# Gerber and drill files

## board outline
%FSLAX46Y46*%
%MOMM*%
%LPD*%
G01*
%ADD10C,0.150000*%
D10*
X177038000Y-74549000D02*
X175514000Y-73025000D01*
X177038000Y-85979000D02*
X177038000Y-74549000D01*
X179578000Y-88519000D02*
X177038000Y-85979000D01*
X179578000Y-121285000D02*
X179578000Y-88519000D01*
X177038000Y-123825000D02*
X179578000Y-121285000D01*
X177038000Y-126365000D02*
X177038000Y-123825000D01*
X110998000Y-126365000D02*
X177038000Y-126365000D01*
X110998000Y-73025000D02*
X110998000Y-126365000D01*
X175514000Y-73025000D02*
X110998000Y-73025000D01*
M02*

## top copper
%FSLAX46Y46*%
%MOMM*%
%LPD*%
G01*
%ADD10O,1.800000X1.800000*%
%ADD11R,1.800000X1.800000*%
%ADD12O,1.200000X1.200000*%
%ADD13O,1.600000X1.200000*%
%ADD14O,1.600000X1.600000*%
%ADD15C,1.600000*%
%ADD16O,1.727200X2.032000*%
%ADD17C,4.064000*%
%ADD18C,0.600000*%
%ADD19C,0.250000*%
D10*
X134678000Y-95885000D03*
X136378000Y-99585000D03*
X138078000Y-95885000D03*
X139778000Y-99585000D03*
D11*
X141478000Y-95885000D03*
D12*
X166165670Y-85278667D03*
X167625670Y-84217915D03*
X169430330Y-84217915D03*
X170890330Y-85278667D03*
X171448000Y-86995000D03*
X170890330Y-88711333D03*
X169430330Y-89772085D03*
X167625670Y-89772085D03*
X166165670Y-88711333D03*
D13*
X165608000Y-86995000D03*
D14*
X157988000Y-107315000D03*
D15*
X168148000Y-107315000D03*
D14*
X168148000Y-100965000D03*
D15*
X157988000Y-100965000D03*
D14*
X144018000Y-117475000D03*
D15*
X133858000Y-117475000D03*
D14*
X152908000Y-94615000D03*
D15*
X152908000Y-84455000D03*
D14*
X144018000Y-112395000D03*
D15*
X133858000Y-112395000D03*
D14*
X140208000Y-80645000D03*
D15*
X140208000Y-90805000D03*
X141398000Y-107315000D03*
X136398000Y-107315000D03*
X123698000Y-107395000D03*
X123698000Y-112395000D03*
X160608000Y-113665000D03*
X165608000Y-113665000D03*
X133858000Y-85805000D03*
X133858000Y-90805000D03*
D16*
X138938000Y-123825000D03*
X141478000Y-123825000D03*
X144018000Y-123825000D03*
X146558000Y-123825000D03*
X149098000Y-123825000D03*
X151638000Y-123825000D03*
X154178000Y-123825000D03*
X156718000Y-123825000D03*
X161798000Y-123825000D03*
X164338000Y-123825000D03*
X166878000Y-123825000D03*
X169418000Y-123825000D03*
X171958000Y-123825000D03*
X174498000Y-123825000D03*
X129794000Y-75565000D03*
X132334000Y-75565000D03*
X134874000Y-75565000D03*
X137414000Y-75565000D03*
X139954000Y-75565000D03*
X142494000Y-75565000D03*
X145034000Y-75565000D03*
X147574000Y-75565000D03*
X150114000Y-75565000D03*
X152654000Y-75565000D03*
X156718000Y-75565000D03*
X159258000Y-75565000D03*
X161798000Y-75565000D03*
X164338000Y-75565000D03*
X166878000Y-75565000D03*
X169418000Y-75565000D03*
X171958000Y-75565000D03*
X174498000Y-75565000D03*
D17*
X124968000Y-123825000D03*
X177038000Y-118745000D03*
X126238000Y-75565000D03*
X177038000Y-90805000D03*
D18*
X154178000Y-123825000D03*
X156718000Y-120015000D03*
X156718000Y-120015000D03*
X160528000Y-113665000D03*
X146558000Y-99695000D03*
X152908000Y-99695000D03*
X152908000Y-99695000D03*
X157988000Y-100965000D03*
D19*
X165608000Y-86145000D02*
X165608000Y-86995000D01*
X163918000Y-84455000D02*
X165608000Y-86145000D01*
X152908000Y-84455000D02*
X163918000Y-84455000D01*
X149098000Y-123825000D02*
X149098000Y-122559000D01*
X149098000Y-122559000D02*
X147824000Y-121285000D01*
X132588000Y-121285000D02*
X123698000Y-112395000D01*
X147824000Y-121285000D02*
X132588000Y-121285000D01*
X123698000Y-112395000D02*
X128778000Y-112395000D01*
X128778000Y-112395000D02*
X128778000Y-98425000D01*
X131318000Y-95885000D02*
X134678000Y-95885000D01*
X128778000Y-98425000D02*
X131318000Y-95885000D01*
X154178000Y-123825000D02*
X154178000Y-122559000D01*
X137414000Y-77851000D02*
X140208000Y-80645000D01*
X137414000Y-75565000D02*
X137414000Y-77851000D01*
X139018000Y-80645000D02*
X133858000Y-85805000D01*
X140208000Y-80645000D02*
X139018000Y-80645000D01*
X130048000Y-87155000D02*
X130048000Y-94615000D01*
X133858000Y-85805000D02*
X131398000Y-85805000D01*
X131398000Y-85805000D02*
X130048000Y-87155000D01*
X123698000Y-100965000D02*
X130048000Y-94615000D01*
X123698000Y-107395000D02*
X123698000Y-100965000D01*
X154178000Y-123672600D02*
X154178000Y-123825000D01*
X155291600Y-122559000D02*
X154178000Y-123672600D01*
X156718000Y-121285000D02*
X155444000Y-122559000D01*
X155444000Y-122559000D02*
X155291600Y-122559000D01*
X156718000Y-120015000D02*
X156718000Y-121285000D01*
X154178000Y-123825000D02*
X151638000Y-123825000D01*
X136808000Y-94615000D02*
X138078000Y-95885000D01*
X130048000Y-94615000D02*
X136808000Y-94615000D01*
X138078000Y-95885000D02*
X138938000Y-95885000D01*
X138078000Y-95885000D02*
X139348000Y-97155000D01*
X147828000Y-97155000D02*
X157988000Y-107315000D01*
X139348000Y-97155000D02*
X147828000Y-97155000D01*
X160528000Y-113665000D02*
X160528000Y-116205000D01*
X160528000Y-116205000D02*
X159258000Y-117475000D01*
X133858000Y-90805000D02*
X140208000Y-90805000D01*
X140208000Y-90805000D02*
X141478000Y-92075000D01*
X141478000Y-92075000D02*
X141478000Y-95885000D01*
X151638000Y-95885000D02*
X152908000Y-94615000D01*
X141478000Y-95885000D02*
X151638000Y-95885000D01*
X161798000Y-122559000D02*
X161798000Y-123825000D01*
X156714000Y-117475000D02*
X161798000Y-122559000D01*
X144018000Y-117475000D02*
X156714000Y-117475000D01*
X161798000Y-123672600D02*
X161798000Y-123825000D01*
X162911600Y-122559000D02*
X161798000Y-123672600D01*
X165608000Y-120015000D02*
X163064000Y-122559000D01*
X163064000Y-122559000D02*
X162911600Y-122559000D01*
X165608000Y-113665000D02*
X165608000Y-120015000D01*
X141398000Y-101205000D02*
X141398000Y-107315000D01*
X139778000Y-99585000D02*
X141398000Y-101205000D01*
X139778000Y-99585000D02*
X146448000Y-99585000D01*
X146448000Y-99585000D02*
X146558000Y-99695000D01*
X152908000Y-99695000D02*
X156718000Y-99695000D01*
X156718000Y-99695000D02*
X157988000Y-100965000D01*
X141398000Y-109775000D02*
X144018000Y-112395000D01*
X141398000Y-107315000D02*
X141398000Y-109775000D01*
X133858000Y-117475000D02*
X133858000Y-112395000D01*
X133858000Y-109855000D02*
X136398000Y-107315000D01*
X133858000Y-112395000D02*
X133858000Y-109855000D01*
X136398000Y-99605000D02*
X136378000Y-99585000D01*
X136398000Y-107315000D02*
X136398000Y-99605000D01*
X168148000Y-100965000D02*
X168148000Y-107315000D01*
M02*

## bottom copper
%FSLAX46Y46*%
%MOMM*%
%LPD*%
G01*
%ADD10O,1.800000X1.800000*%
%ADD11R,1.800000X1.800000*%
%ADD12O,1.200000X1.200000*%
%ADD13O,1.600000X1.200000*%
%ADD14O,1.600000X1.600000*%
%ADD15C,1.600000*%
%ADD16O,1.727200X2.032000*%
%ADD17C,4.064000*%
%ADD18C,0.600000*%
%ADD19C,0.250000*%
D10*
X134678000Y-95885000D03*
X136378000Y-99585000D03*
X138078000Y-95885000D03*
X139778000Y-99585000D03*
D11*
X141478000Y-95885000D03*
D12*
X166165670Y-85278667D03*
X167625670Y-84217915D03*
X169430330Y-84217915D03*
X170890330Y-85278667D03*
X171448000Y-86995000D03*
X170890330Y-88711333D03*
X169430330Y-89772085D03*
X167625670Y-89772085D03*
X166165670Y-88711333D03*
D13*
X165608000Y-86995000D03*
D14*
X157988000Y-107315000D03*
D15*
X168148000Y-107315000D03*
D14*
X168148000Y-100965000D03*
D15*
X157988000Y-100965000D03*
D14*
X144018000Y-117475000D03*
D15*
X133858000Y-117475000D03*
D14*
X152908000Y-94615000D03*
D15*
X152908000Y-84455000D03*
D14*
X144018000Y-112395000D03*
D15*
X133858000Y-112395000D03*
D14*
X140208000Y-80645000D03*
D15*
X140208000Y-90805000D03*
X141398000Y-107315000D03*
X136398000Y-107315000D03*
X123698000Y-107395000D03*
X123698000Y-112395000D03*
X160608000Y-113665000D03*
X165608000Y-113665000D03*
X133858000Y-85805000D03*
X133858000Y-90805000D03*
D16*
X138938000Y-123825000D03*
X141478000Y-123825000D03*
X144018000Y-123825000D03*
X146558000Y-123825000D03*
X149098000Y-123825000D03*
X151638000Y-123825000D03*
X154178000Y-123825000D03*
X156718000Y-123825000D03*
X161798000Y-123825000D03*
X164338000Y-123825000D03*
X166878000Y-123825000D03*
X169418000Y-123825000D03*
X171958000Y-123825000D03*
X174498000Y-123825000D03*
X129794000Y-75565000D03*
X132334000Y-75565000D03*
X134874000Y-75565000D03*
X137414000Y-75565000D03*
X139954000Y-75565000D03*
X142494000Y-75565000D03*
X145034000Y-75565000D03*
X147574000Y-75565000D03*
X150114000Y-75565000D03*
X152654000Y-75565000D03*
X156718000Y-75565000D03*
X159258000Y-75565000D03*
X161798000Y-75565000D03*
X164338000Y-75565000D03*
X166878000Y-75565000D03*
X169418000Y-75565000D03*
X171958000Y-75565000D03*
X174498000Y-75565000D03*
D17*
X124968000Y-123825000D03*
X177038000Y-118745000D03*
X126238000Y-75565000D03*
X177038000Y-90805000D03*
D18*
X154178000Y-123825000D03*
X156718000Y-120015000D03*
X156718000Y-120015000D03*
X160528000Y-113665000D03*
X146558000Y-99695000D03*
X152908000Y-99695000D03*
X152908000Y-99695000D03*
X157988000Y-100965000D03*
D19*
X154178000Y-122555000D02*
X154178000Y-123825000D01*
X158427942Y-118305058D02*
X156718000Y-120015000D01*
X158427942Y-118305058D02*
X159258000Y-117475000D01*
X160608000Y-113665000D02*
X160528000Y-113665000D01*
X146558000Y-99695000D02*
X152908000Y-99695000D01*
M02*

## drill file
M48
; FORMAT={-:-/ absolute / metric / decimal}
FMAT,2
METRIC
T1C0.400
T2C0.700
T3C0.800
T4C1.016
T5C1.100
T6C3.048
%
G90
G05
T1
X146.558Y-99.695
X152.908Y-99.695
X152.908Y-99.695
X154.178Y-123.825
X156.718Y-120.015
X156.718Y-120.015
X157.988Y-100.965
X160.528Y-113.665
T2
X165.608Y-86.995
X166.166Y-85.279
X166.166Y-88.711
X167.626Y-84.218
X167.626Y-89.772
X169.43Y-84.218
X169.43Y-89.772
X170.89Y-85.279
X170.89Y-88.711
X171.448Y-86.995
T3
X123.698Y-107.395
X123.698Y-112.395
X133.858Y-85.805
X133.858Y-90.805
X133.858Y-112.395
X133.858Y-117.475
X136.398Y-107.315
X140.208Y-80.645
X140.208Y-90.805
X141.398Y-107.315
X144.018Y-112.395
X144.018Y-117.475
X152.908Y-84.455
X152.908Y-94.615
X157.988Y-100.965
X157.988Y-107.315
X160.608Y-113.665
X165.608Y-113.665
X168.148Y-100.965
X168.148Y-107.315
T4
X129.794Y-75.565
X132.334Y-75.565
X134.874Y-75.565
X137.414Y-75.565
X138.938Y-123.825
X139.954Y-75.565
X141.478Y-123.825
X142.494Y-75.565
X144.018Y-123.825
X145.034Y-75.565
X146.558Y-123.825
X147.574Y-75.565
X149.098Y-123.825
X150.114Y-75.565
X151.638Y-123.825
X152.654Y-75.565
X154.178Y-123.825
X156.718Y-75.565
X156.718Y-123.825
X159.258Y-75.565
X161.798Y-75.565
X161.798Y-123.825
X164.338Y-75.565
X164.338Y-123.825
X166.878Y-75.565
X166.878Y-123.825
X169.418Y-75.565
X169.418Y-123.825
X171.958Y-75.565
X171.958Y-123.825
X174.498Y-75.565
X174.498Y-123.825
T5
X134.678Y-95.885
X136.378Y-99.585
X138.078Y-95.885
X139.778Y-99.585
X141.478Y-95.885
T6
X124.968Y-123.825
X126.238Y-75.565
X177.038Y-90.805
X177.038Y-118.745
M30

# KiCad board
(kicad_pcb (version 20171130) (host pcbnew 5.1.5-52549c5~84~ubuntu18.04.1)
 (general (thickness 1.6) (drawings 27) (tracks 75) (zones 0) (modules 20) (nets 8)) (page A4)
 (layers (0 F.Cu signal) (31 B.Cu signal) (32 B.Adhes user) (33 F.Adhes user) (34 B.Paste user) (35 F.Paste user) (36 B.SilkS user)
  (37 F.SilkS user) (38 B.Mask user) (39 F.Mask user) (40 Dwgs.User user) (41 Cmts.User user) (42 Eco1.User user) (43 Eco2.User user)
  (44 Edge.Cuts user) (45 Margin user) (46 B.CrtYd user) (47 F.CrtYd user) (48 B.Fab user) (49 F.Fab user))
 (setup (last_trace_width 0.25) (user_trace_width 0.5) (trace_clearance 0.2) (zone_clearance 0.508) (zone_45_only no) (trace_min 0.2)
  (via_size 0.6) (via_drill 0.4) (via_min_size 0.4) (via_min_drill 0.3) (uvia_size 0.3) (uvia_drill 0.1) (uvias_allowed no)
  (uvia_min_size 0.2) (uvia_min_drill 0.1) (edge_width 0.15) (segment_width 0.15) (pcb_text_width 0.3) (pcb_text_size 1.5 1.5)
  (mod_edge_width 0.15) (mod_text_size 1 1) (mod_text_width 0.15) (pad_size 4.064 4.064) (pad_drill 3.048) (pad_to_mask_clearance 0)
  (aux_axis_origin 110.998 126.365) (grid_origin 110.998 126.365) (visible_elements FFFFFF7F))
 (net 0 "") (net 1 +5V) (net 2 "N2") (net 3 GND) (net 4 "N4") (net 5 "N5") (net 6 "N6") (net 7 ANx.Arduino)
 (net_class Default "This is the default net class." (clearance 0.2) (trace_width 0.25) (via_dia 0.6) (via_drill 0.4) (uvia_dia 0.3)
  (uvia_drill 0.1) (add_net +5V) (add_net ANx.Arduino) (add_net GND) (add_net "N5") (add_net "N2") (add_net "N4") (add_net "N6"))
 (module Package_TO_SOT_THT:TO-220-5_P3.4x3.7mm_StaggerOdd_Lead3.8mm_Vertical (layer F.Cu) (at 141.478 95.885 180)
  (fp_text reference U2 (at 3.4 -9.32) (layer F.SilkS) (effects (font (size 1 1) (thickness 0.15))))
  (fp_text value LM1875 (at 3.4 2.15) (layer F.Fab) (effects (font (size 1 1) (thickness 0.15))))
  (pad 5 thru_hole oval (at 6.8 0 180) (size 1.8 1.8) (drill 1.1) (layers *.Cu *.Mask) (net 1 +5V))
  (pad 4 thru_hole oval (at 5.1 -3.7 180) (size 1.8 1.8) (drill 1.1) (layers *.Cu *.Mask) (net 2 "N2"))
  (pad 3 thru_hole oval (at 3.4 0 180) (size 1.8 1.8) (drill 1.1) (layers *.Cu *.Mask) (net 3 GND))
  (pad 2 thru_hole oval (at 1.7 -3.7 180) (size 1.8 1.8) (drill 1.1) (layers *.Cu *.Mask) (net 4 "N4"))
  (pad 1 thru_hole rect (at 0 0 180) (size 1.8 1.8) (drill 1.1) (layers *.Cu *.Mask) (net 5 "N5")))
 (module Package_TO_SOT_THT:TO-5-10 (layer F.Cu) (at 165.608 86.995)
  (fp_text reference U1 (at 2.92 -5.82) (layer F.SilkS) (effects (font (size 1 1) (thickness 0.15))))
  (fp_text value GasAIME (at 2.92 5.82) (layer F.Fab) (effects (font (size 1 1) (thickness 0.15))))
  (pad 10 thru_hole oval (at 0.55767 -1.716333) (size 1.2 1.2) (drill 0.7) (layers *.Cu *.Mask))
  (pad 9 thru_hole oval (at 2.01767 -2.777085) (size 1.2 1.2) (drill 0.7) (layers *.Cu *.Mask))
  (pad 8 thru_hole oval (at 3.82233 -2.777085) (size 1.2 1.2) (drill 0.7) (layers *.Cu *.Mask))
  (pad 7 thru_hole oval (at 5.28233 -1.716333) (size 1.2 1.2) (drill 0.7) (layers *.Cu *.Mask))
  (pad 6 thru_hole oval (at 5.84 0) (size 1.2 1.2) (drill 0.7) (layers *.Cu *.Mask))
  (pad 5 thru_hole oval (at 5.28233 1.716333) (size 1.2 1.2) (drill 0.7) (layers *.Cu *.Mask))
  (pad 4 thru_hole oval (at 3.82233 2.777085) (size 1.2 1.2) (drill 0.7) (layers *.Cu *.Mask))
  (pad 3 thru_hole oval (at 2.01767 2.777085) (size 1.2 1.2) (drill 0.7) (layers *.Cu *.Mask))
  (pad 2 thru_hole oval (at 0.55767 1.716333) (size 1.2 1.2) (drill 0.7) (layers *.Cu *.Mask))
  (pad 1 thru_hole oval (at 0 0) (size 1.6 1.2) (drill 0.7) (layers *.Cu *.Mask)))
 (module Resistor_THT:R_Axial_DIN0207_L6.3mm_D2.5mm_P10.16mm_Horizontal (layer F.Cu) (at 168.148 107.315 180)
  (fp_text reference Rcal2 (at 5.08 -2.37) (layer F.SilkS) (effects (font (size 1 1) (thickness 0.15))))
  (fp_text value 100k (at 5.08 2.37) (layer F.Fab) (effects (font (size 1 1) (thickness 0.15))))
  (pad 2 thru_hole oval (at 10.16 0 180) (size 1.6 1.6) (drill 0.8) (layers *.Cu *.Mask) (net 3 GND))
  (pad 1 thru_hole circle (at 0 0 180) (size 1.6 1.6) (drill 0.8) (layers *.Cu *.Mask) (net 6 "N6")))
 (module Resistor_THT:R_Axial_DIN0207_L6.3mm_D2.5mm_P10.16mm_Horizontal (layer F.Cu) (at 157.988 100.965)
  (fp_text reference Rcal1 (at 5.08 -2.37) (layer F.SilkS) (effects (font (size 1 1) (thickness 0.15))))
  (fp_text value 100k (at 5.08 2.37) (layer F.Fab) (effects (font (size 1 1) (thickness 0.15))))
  (pad 2 thru_hole oval (at 10.16 0) (size 1.6 1.6) (drill 0.8) (layers *.Cu *.Mask) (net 6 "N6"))
  (pad 1 thru_hole circle (at 0 0) (size 1.6 1.6) (drill 0.8) (layers *.Cu *.Mask) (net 4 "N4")))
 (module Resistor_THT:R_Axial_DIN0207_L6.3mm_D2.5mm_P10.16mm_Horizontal (layer F.Cu) (at 133.858 117.475)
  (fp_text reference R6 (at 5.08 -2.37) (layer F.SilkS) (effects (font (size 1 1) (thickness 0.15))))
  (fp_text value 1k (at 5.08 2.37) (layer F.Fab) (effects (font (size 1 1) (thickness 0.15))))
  (pad 2 thru_hole oval (at 10.16 0) (size 1.6 1.6) (drill 0.8) (layers *.Cu *.Mask) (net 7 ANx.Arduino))
  (pad 1 thru_hole circle (at 0 0) (size 1.6 1.6) (drill 0.8) (layers *.Cu *.Mask) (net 2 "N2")))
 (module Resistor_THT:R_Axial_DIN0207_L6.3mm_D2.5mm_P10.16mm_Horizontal (layer F.Cu) (at 152.908 84.455 270)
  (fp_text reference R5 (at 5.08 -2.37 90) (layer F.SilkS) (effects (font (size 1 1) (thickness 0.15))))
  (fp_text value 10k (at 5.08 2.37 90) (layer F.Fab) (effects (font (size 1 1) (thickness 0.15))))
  (pad 2 thru_hole oval (at 10.16 0 270) (size 1.6 1.6) (drill 0.8) (layers *.Cu *.Mask) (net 5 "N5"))
  (pad 1 thru_hole circle (at 0 0 270) (size 1.6 1.6) (drill 0.8) (layers *.Cu *.Mask)))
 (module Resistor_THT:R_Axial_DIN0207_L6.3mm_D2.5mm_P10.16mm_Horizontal (layer F.Cu) (at 133.858 112.395)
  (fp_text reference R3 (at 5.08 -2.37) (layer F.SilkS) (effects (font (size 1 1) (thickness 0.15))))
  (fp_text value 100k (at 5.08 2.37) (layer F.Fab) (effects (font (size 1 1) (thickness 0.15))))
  (pad 2 thru_hole oval (at 10.16 0) (size 1.6 1.6) (drill 0.8) (layers *.Cu *.Mask) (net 4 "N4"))
  (pad 1 thru_hole circle (at 0 0) (size 1.6 1.6) (drill 0.8) (layers *.Cu *.Mask) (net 2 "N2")))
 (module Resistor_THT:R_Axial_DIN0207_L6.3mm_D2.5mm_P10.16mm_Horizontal (layer F.Cu) (at 140.208 90.805 90)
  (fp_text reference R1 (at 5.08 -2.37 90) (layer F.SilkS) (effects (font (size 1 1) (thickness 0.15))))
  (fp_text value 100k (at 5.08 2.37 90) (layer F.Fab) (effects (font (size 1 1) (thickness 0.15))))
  (pad 2 thru_hole oval (at 10.16 0 90) (size 1.6 1.6) (drill 0.8) (layers *.Cu *.Mask) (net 3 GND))
  (pad 1 thru_hole circle (at 0 0 90) (size 1.6 1.6) (drill 0.8) (layers *.Cu *.Mask) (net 5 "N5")))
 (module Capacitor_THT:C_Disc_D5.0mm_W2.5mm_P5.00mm (layer F.Cu) (at 136.398 107.315)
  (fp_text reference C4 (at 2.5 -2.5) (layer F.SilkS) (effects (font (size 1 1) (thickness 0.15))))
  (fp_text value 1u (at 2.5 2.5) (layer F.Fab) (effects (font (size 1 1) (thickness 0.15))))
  (pad 2 thru_hole circle (at 5 0) (size 1.6 1.6) (drill 0.8) (layers *.Cu *.Mask) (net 4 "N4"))
  (pad 1 thru_hole circle (at 0 0) (size 1.6 1.6) (drill 0.8) (layers *.Cu *.Mask) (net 2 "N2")))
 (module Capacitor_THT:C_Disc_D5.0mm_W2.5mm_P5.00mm (layer F.Cu) (at 123.698 112.395 90)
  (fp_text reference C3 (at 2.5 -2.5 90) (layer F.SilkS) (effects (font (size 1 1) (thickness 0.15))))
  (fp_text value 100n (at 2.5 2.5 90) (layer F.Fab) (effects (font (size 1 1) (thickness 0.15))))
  (pad 2 thru_hole circle (at 5 0 90) (size 1.6 1.6) (drill 0.8) (layers *.Cu *.Mask) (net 3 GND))
  (pad 1 thru_hole circle (at 0 0 90) (size 1.6 1.6) (drill 0.8) (layers *.Cu *.Mask) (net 1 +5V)))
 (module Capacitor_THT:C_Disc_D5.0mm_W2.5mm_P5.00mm (layer F.Cu) (at 165.608 113.665 180)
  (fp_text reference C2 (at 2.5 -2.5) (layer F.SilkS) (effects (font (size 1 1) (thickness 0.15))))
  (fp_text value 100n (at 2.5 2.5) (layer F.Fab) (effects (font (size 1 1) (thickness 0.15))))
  (pad 2 thru_hole circle (at 5 0 180) (size 1.6 1.6) (drill 0.8) (layers *.Cu *.Mask) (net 3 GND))
  (pad 1 thru_hole circle (at 0 0 180) (size 1.6 1.6) (drill 0.8) (layers *.Cu *.Mask) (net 7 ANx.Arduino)))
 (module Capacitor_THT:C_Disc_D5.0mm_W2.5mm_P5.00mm (layer F.Cu) (at 133.858 90.805 90)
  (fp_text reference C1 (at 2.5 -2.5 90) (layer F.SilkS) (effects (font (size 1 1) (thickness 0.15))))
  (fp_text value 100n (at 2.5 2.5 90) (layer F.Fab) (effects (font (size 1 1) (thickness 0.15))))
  (pad 2 thru_hole circle (at 5 0 90) (size 1.6 1.6) (drill 0.8) (layers *.Cu *.Mask) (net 3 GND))
  (pad 1 thru_hole circle (at 0 0 90) (size 1.6 1.6) (drill 0.8) (layers *.Cu *.Mask) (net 5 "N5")))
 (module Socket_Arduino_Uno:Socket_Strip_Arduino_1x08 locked (layer F.Cu) (at 138.938 123.825)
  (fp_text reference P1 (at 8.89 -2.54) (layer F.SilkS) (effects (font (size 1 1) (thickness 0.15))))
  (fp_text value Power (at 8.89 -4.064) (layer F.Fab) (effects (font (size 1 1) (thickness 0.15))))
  (pad 1 thru_hole oval (at 0 0) (size 1.7272 2.032) (drill 1.016) (layers *.Cu *.Mask F.SilkS))
  (pad 2 thru_hole oval (at 2.54 0) (size 1.7272 2.032) (drill 1.016) (layers *.Cu *.Mask F.SilkS))
  (pad 3 thru_hole oval (at 5.08 0) (size 1.7272 2.032) (drill 1.016) (layers *.Cu *.Mask F.SilkS))
  (pad 4 thru_hole oval (at 7.62 0) (size 1.7272 2.032) (drill 1.016) (layers *.Cu *.Mask F.SilkS))
  (pad 5 thru_hole oval (at 10.16 0) (size 1.7272 2.032) (drill 1.016) (layers *.Cu *.Mask F.SilkS) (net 1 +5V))
  (pad 6 thru_hole oval (at 12.7 0) (size 1.7272 2.032) (drill 1.016) (layers *.Cu *.Mask F.SilkS) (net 3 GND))
  (pad 7 thru_hole oval (at 15.24 0) (size 1.7272 2.032) (drill 1.016) (layers *.Cu *.Mask F.SilkS) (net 3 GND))
  (pad 8 thru_hole oval (at 17.78 0) (size 1.7272 2.032) (drill 1.016) (layers *.Cu *.Mask F.SilkS)))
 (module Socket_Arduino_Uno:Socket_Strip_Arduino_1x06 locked (layer F.Cu) (at 161.798 123.825)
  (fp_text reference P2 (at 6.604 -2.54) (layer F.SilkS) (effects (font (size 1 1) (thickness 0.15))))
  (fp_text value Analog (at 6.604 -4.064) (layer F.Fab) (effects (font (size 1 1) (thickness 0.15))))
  (pad 1 thru_hole oval (at 0 0) (size 1.7272 2.032) (drill 1.016) (layers *.Cu *.Mask F.SilkS) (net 7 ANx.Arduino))
  (pad 2 thru_hole oval (at 2.54 0) (size 1.7272 2.032) (drill 1.016) (layers *.Cu *.Mask F.SilkS))
  (pad 3 thru_hole oval (at 5.08 0) (size 1.7272 2.032) (drill 1.016) (layers *.Cu *.Mask F.SilkS))
  (pad 4 thru_hole oval (at 7.62 0) (size 1.7272 2.032) (drill 1.016) (layers *.Cu *.Mask F.SilkS))
  (pad 5 thru_hole oval (at 10.16 0) (size 1.7272 2.032) (drill 1.016) (layers *.Cu *.Mask F.SilkS))
  (pad 6 thru_hole oval (at 12.7 0) (size 1.7272 2.032) (drill 1.016) (layers *.Cu *.Mask F.SilkS)))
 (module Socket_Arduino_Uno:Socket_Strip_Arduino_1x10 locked (layer F.Cu) (at 129.794 75.565)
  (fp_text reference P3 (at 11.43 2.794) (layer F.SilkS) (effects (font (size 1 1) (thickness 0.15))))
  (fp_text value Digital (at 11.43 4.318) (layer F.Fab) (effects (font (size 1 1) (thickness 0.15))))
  (pad 1 thru_hole oval (at 0 0) (size 1.7272 2.032) (drill 1.016) (layers *.Cu *.Mask F.SilkS))
  (pad 2 thru_hole oval (at 2.54 0) (size 1.7272 2.032) (drill 1.016) (layers *.Cu *.Mask F.SilkS))
  (pad 3 thru_hole oval (at 5.08 0) (size 1.7272 2.032) (drill 1.016) (layers *.Cu *.Mask F.SilkS))
  (pad 4 thru_hole oval (at 7.62 0) (size 1.7272 2.032) (drill 1.016) (layers *.Cu *.Mask F.SilkS) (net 3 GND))
  (pad 5 thru_hole oval (at 10.16 0) (size 1.7272 2.032) (drill 1.016) (layers *.Cu *.Mask F.SilkS))
  (pad 6 thru_hole oval (at 12.7 0) (size 1.7272 2.032) (drill 1.016) (layers *.Cu *.Mask F.SilkS))
  (pad 7 thru_hole oval (at 15.24 0) (size 1.7272 2.032) (drill 1.016) (layers *.Cu *.Mask F.SilkS))
  (pad 8 thru_hole oval (at 17.78 0) (size 1.7272 2.032) (drill 1.016) (layers *.Cu *.Mask F.SilkS))
  (pad 9 thru_hole oval (at 20.32 0) (size 1.7272 2.032) (drill 1.016) (layers *.Cu *.Mask F.SilkS))
  (pad 10 thru_hole oval (at 22.86 0) (size 1.7272 2.032) (drill 1.016) (layers *.Cu *.Mask F.SilkS)))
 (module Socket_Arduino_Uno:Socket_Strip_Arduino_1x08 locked (layer F.Cu) (at 156.718 75.565)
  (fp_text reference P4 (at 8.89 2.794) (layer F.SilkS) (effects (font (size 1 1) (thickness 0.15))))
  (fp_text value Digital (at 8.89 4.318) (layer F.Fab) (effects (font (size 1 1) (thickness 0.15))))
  (pad 1 thru_hole oval (at 0 0) (size 1.7272 2.032) (drill 1.016) (layers *.Cu *.Mask F.SilkS))
  (pad 2 thru_hole oval (at 2.54 0) (size 1.7272 2.032) (drill 1.016) (layers *.Cu *.Mask F.SilkS))
  (pad 3 thru_hole oval (at 5.08 0) (size 1.7272 2.032) (drill 1.016) (layers *.Cu *.Mask F.SilkS))
  (pad 4 thru_hole oval (at 7.62 0) (size 1.7272 2.032) (drill 1.016) (layers *.Cu *.Mask F.SilkS))
  (pad 5 thru_hole oval (at 10.16 0) (size 1.7272 2.032) (drill 1.016) (layers *.Cu *.Mask F.SilkS))
  (pad 6 thru_hole oval (at 12.7 0) (size 1.7272 2.032) (drill 1.016) (layers *.Cu *.Mask F.SilkS))
  (pad 7 thru_hole oval (at 15.24 0) (size 1.7272 2.032) (drill 1.016) (layers *.Cu *.Mask F.SilkS))
  (pad 8 thru_hole oval (at 17.78 0) (size 1.7272 2.032) (drill 1.016) (layers *.Cu *.Mask F.SilkS)))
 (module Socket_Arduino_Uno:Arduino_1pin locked (layer F.Cu) (at 124.968 123.825)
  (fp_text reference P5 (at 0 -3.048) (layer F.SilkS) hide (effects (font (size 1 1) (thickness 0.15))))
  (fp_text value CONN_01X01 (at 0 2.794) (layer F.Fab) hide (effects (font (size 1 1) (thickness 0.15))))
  (pad 1 thru_hole circle (at 0 0) (size 4.064 4.064) (drill 3.048) (layers *.Cu *.Mask F.SilkS)))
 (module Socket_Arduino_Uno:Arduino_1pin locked (layer F.Cu) (at 177.038 118.745)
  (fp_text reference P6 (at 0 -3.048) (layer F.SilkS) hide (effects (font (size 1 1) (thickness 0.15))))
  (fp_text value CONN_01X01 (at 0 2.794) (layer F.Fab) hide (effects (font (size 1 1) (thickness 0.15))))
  (pad 1 thru_hole circle (at 0 0) (size 4.064 4.064) (drill 3.048) (layers *.Cu *.Mask F.SilkS)))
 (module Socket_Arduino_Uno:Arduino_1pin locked (layer F.Cu) (at 126.238 75.565)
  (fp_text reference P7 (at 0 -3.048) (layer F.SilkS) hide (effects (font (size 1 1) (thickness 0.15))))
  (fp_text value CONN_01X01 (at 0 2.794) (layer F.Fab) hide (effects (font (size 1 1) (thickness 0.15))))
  (pad 1 thru_hole circle (at 0 0) (size 4.064 4.064) (drill 3.048) (layers *.Cu *.Mask F.SilkS)))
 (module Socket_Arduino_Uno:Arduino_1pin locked (layer F.Cu) (at 177.038 90.805)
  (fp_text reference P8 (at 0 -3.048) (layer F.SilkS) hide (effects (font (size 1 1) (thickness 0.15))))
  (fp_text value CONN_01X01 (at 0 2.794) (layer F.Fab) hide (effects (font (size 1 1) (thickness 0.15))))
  (pad 1 thru_hole circle (at 0 0) (size 4.064 4.064) (drill 3.048) (layers *.Cu *.Mask F.SilkS)))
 (gr_line (start 177.038 74.549) (end 175.514 73.025) (angle 90) (layer Edge.Cuts) (width 0.15))
 (gr_line (start 177.038 85.979) (end 177.038 74.549) (angle 90) (layer Edge.Cuts) (width 0.15))
 (gr_line (start 179.578 88.519) (end 177.038 85.979) (angle 90) (layer Edge.Cuts) (width 0.15))
 (gr_line (start 179.578 121.285) (end 179.578 88.519) (angle 90) (layer Edge.Cuts) (width 0.15))
 (gr_line (start 177.038 123.825) (end 179.578 121.285) (angle 90) (layer Edge.Cuts) (width 0.15))
 (gr_line (start 177.038 126.365) (end 177.038 123.825) (angle 90) (layer Edge.Cuts) (width 0.15))
 (gr_line (start 110.998 126.365) (end 177.038 126.365) (angle 90) (layer Edge.Cuts) (width 0.15))
 (gr_line (start 110.998 73.025) (end 110.998 126.365) (angle 90) (layer Edge.Cuts) (width 0.15))
 (gr_line (start 175.514 73.025) (end 110.998 73.025) (angle 90) (layer Edge.Cuts) (width 0.15))
 (segment (start 165.608 86.145) (end 165.608 86.995) (width 0.25) (layer F.Cu) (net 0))
 (segment (start 163.918 84.455) (end 165.608 86.145) (width 0.25) (layer F.Cu) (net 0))
 (segment (start 152.908 84.455) (end 163.918 84.455) (width 0.25) (layer F.Cu) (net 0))
 (segment (start 149.098 123.825) (end 149.098 122.559) (width 0.25) (layer F.Cu) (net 1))
 (segment (start 149.098 122.559) (end 147.824 121.285) (width 0.25) (layer F.Cu) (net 1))
 (segment (start 132.588 121.285) (end 123.698 112.395) (width 0.25) (layer F.Cu) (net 1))
 (segment (start 147.824 121.285) (end 132.588 121.285) (width 0.25) (layer F.Cu) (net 1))
 (segment (start 123.698 112.395) (end 128.778 112.395) (width 0.25) (layer F.Cu) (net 1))
 (segment (start 128.778 112.395) (end 128.778 98.425) (width 0.25) (layer F.Cu) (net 1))
 (segment (start 131.318 95.885) (end 134.678 95.885) (width 0.25) (layer F.Cu) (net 1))
 (segment (start 128.778 98.425) (end 131.318 95.885) (width 0.25) (layer F.Cu) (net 1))
 (segment (start 154.178 123.825) (end 154.178 122.559) (width 0.25) (layer F.Cu) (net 3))
 (segment (start 137.414 77.851) (end 140.208 80.645) (width 0.25) (layer F.Cu) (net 3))
 (segment (start 137.414 75.565) (end 137.414 77.851) (width 0.25) (layer F.Cu) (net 3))
 (segment (start 139.018 80.645) (end 133.858 85.805) (width 0.25) (layer F.Cu) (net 3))
 (segment (start 140.208 80.645) (end 139.018 80.645) (width 0.25) (layer F.Cu) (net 3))
 (segment (start 130.048 87.155) (end 130.048 94.615) (width 0.25) (layer F.Cu) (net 3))
 (segment (start 133.858 85.805) (end 131.398 85.805) (width 0.25) (layer F.Cu) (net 3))
 (segment (start 131.398 85.805) (end 130.048 87.155) (width 0.25) (layer F.Cu) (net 3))
 (segment (start 123.698 100.965) (end 130.048 94.615) (width 0.25) (layer F.Cu) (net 3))
 (segment (start 123.698 107.395) (end 123.698 100.965) (width 0.25) (layer F.Cu) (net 3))
 (segment (start 154.178 122.555) (end 154.178 123.825) (width 0.25) (layer B.Cu) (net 3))
 (via (at 154.178 123.825) (size 0.6) (drill 0.4) (layers F.Cu B.Cu) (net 3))
 (segment (start 158.427942 118.305058) (end 156.718 120.015) (width 0.25) (layer B.Cu) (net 3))
 (via (at 156.718 120.015) (size 0.6) (drill 0.4) (layers F.Cu B.Cu) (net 3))
 (via (at 156.718 120.015) (size 0.6) (drill 0.4) (layers F.Cu B.Cu) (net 3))
 (segment (start 154.178 123.6726) (end 154.178 123.825) (width 0.25) (layer F.Cu) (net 3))
 (segment (start 155.2916 122.559) (end 154.178 123.6726) (width 0.25) (layer F.Cu) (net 3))
 (segment (start 156.718 121.285) (end 155.444 122.559) (width 0.25) (layer F.Cu) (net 3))
 (segment (start 155.444 122.559) (end 155.2916 122.559) (width 0.25) (layer F.Cu) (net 3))
 (segment (start 156.718 120.015) (end 156.718 121.285) (width 0.25) (layer F.Cu) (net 3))
 (segment (start 154.178 123.825) (end 151.638 123.825) (width 0.25) (layer F.Cu) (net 3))
 (segment (start 136.808 94.615) (end 138.078 95.885) (width 0.25) (layer F.Cu) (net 3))
 (segment (start 130.048 94.615) (end 136.808 94.615) (width 0.25) (layer F.Cu) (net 3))
 (segment (start 138.078 95.885) (end 138.938 95.885) (width 0.25) (layer F.Cu) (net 3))
 (segment (start 138.078 95.885) (end 139.348 97.155) (width 0.25) (layer F.Cu) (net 3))
 (segment (start 147.828 97.155) (end 157.988 107.315) (width 0.25) (layer F.Cu) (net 3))
 (segment (start 139.348 97.155) (end 147.828 97.155) (width 0.25) (layer F.Cu) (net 3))
 (segment (start 158.427942 118.305058) (end 159.258 117.475) (width 0.25) (layer B.Cu) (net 3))
 (via (at 160.528 113.665) (size 0.6) (drill 0.4) (layers F.Cu B.Cu) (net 3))
 (segment (start 160.608 113.665) (end 160.528 113.665) (width 0.25) (layer B.Cu) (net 3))
 (segment (start 160.528 113.665) (end 160.528 116.205) (width 0.25) (layer F.Cu) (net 3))
 (segment (start 160.528 116.205) (end 159.258 117.475) (width 0.25) (layer F.Cu) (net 3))
 (segment (start 133.858 90.805) (end 140.208 90.805) (width 0.25) (layer F.Cu) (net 5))
 (segment (start 140.208 90.805) (end 141.478 92.075) (width 0.25) (layer F.Cu) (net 5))
 (segment (start 141.478 92.075) (end 141.478 95.885) (width 0.25) (layer F.Cu) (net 5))
 (segment (start 151.638 95.885) (end 152.908 94.615) (width 0.25) (layer F.Cu) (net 5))
 (segment (start 141.478 95.885) (end 151.638 95.885) (width 0.25) (layer F.Cu) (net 5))
 (segment (start 161.798 122.559) (end 161.798 123.825) (width 0.25) (layer F.Cu) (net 7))
 (segment (start 156.714 117.475) (end 161.798 122.559) (width 0.25) (layer F.Cu) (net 7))
 (segment (start 144.018 117.475) (end 156.714 117.475) (width 0.25) (layer F.Cu) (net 7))
 (segment (start 161.798 123.6726) (end 161.798 123.825) (width 0.25) (layer F.Cu) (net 7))
 (segment (start 162.9116 122.559) (end 161.798 123.6726) (width 0.25) (layer F.Cu) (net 7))
 (segment (start 165.608 120.015) (end 163.064 122.559) (width 0.25) (layer F.Cu) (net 7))
 (segment (start 163.064 122.559) (end 162.9116 122.559) (width 0.25) (layer F.Cu) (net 7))
 (segment (start 165.608 113.665) (end 165.608 120.015) (width 0.25) (layer F.Cu) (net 7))
 (segment (start 141.398 101.205) (end 141.398 107.315) (width 0.25) (layer F.Cu) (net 4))
 (segment (start 139.778 99.585) (end 141.398 101.205) (width 0.25) (layer F.Cu) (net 4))
 (segment (start 139.778 99.585) (end 146.448 99.585) (width 0.25) (layer F.Cu) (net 4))
 (via (at 146.558 99.695) (size 0.6) (drill 0.4) (layers F.Cu B.Cu) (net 4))
 (segment (start 146.448 99.585) (end 146.558 99.695) (width 0.25) (layer F.Cu) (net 4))
 (segment (start 146.558 99.695) (end 152.908 99.695) (width 0.25) (layer B.Cu) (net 4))
 (via (at 152.908 99.695) (size 0.6) (drill 0.4) (layers F.Cu B.Cu) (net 4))
 (via (at 152.908 99.695) (size 0.6) (drill 0.4) (layers F.Cu B.Cu) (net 4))
 (via (at 157.988 100.965) (size 0.6) (drill 0.4) (layers F.Cu B.Cu) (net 4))
 (segment (start 152.908 99.695) (end 156.718 99.695) (width 0.25) (layer F.Cu) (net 4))
 (segment (start 156.718 99.695) (end 157.988 100.965) (width 0.25) (layer F.Cu) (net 4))
 (segment (start 141.398 109.775) (end 144.018 112.395) (width 0.25) (layer F.Cu) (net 4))
 (segment (start 141.398 107.315) (end 141.398 109.775) (width 0.25) (layer F.Cu) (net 4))
 (segment (start 133.858 117.475) (end 133.858 112.395) (width 0.25) (layer F.Cu) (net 2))
 (segment (start 133.858 109.855) (end 136.398 107.315) (width 0.25) (layer F.Cu) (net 2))
 (segment (start 133.858 112.395) (end 133.858 109.855) (width 0.25) (layer F.Cu) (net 2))
 (segment (start 136.398 99.605) (end 136.378 99.585) (width 0.25) (layer F.Cu) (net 2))
 (segment (start 136.398 107.315) (end 136.398 99.605) (width 0.25) (layer F.Cu) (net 2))
 (segment (start 168.148 100.965) (end 168.148 107.315) (width 0.25) (layer F.Cu) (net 6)))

